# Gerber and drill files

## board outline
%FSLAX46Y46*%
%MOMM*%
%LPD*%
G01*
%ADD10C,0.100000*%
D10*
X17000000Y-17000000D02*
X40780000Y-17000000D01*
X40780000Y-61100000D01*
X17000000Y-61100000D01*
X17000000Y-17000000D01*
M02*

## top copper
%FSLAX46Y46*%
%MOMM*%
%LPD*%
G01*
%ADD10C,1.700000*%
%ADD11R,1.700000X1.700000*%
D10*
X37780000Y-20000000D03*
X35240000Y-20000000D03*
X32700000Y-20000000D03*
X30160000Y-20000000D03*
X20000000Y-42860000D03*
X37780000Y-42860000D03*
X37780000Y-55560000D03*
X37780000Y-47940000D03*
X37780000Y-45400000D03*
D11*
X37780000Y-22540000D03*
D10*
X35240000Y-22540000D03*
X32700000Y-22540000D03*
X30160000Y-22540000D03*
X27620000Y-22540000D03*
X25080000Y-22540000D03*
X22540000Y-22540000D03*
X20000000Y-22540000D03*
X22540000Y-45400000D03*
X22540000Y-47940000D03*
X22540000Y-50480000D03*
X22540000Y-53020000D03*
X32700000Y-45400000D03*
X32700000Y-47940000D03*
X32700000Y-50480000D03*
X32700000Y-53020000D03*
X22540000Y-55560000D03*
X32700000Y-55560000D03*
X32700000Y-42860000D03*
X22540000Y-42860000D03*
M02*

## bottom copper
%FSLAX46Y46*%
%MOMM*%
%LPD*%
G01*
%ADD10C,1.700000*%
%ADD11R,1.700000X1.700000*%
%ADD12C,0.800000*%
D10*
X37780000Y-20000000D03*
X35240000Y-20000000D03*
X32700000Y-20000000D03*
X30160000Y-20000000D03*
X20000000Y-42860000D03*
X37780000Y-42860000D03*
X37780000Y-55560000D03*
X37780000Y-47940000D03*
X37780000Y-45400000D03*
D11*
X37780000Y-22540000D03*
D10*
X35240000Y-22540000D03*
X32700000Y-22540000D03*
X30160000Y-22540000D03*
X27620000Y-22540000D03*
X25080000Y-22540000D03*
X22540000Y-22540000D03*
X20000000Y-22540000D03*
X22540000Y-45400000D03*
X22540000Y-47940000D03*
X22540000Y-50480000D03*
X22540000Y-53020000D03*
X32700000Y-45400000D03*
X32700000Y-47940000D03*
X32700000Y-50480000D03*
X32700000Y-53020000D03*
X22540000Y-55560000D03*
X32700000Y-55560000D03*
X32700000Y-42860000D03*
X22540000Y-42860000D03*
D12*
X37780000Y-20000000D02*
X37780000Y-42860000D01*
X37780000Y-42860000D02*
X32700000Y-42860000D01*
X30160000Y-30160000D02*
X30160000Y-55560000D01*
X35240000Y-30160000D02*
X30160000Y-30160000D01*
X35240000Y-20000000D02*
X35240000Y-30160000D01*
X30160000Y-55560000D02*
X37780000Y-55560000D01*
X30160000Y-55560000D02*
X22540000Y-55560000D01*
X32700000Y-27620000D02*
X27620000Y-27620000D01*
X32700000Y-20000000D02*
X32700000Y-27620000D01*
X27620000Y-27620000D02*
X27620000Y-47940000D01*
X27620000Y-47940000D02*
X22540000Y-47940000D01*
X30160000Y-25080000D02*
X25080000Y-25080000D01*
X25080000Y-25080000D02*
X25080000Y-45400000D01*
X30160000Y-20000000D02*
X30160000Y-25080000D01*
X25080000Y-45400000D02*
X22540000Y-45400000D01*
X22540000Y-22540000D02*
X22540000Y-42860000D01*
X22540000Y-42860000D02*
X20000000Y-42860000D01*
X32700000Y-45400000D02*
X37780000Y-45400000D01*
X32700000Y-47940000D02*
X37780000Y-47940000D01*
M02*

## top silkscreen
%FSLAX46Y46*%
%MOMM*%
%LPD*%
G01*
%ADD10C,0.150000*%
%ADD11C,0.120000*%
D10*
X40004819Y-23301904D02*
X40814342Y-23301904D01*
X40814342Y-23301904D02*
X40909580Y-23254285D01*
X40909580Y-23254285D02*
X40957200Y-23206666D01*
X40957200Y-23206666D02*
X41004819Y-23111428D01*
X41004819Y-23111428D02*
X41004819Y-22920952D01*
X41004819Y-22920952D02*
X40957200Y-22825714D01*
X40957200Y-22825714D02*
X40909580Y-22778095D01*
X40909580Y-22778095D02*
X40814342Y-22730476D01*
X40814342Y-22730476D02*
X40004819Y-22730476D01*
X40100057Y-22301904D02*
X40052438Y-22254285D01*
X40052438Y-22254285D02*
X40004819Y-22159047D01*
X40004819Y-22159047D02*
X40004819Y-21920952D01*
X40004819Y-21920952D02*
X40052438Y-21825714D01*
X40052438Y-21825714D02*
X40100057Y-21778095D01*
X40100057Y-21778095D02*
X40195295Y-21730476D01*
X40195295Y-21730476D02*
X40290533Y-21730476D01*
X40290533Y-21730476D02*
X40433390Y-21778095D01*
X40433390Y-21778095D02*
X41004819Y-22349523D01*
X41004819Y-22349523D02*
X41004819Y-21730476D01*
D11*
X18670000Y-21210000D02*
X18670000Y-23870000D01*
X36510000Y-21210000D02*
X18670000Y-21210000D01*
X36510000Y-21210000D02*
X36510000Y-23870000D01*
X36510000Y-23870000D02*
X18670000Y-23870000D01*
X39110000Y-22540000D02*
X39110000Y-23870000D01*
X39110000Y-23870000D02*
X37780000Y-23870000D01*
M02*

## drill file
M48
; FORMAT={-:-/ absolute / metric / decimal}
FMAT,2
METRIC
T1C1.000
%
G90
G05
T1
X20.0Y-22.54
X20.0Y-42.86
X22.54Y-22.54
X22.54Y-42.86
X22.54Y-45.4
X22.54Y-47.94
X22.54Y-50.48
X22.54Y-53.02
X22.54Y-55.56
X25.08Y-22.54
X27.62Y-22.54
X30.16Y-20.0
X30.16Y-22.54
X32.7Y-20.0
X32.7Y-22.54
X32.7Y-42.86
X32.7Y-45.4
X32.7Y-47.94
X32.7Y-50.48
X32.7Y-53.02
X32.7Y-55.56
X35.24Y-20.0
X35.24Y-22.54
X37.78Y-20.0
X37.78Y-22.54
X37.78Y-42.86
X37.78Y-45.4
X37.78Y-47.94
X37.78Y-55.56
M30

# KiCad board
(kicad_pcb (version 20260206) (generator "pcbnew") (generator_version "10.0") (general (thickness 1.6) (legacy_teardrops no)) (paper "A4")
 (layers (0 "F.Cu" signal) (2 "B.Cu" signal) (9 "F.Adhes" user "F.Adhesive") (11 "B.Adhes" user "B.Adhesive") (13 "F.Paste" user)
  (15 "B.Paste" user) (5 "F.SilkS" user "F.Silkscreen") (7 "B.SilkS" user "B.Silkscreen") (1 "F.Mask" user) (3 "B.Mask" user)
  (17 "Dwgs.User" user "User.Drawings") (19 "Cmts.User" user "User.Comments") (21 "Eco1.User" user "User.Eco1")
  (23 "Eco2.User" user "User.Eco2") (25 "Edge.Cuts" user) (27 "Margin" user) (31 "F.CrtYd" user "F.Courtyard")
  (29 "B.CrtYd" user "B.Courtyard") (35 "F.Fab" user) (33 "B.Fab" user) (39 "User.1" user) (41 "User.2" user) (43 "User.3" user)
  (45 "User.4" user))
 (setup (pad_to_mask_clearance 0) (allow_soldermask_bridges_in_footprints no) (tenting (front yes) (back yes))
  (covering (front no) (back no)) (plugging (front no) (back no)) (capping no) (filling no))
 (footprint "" (layer "F.Cu") (at 30.16 20)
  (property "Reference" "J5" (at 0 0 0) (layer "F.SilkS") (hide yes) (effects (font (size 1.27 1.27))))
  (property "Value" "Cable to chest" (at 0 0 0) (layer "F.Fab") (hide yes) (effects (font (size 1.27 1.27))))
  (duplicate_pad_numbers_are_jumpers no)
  (pad "c5V" thru_hole circle (at 7.62 0) (size 1.7 1.7) (drill 1) (layers "*.Cu" "*.Mask") (remove_unused_layers no) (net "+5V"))
  (pad "cGND" thru_hole circle (at 5.08 0) (size 1.7 1.7) (drill 1) (layers "*.Cu" "*.Mask") (remove_unused_layers no) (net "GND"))
  (pad "cSCL" thru_hole circle (at 2.54 0) (size 1.7 1.7) (drill 1) (layers "*.Cu" "*.Mask") (remove_unused_layers no) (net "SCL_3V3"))
  (pad "cSDA" thru_hole circle (at 0 0) (size 1.7 1.7) (drill 1) (layers "*.Cu" "*.Mask") (remove_unused_layers no) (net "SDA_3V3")))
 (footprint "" (layer "F.Cu") (at 20 42.86)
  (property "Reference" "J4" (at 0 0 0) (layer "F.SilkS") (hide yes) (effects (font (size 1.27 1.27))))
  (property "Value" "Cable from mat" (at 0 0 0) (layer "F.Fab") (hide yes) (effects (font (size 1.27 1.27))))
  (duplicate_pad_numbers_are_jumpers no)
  (pad "m3V3" thru_hole circle (at 0 0) (size 1.7 1.7) (drill 1) (layers "*.Cu" "*.Mask") (remove_unused_layers no) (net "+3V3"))
  (pad "m5V" thru_hole circle (at 17.78 0) (size 1.7 1.7) (drill 1) (layers "*.Cu" "*.Mask") (remove_unused_layers no) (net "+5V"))
  (pad "mGND" thru_hole circle (at 17.78 12.7) (size 1.7 1.7) (drill 1) (layers "*.Cu" "*.Mask") (remove_unused_layers no) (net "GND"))
  (pad "mSCL" thru_hole circle (at 17.78 5.08) (size 1.7 1.7) (drill 1) (layers "*.Cu" "*.Mask") (remove_unused_layers no) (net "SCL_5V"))
  (pad "mSDA" thru_hole circle (at 17.78 2.54) (size 1.7 1.7) (drill 1) (layers "*.Cu" "*.Mask") (remove_unused_layers no) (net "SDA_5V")))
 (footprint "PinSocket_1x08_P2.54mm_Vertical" (layer "F.Cu") (at 37.78 22.54 -90)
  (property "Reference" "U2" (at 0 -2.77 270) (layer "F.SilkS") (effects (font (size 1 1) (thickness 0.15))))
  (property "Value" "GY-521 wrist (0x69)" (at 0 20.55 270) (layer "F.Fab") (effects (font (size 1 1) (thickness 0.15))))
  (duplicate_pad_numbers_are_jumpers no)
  (fp_line (start -1.33 19.11) (end 1.33 19.11) (stroke (width 0.12) (type solid)) (layer "F.SilkS"))
  (fp_line (start -1.33 1.27) (end -1.33 19.11) (stroke (width 0.12) (type solid)) (layer "F.SilkS"))
  (fp_line (start -1.33 1.27) (end 1.33 1.27) (stroke (width 0.12) (type solid)) (layer "F.SilkS"))
  (fp_line (start 1.33 1.27) (end 1.33 19.11) (stroke (width 0.12) (type solid)) (layer "F.SilkS"))
  (fp_line (start 0 -1.33) (end 1.33 -1.33) (stroke (width 0.12) (type solid)) (layer "F.SilkS"))
  (fp_line (start 1.33 -1.33) (end 1.33 0) (stroke (width 0.12) (type solid)) (layer "F.SilkS"))
  (pad "1" thru_hole rect (at 0 0 270) (size 1.7 1.7) (drill 1) (layers "*.Cu" "*.Mask") (remove_unused_layers no) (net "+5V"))
  (pad "2" thru_hole circle (at 0 2.54 270) (size 1.7 1.7) (drill 1) (layers "*.Cu" "*.Mask") (remove_unused_layers no) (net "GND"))
  (pad "3" thru_hole circle (at 0 5.08 270) (size 1.7 1.7) (drill 1) (layers "*.Cu" "*.Mask") (remove_unused_layers no) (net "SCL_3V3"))
  (pad "4" thru_hole circle (at 0 7.62 270) (size 1.7 1.7) (drill 1) (layers "*.Cu" "*.Mask") (remove_unused_layers no) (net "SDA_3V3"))
  (pad "5" thru_hole circle (at 0 10.16 270) (size 1.7 1.7) (drill 1) (layers "*.Cu" "*.Mask") (remove_unused_layers no))
  (pad "6" thru_hole circle (at 0 12.7 270) (size 1.7 1.7) (drill 1) (layers "*.Cu" "*.Mask") (remove_unused_layers no))
  (pad "7" thru_hole circle (at 0 15.24 270) (size 1.7 1.7) (drill 1) (layers "*.Cu" "*.Mask") (remove_unused_layers no) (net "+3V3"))
  (pad "8" thru_hole circle (at 0 17.78 270) (size 1.7 1.7) (drill 1) (layers "*.Cu" "*.Mask") (remove_unused_layers no)))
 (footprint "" (layer "F.Cu") (at 22.54 42.86)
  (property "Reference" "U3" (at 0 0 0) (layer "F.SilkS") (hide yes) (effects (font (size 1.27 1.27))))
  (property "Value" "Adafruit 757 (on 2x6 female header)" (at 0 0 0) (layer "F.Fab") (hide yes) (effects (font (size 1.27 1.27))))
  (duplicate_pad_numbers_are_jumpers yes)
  (pad "A1" thru_hole circle (at 0 2.54) (size 1.7 1.7) (drill 1) (layers "*.Cu" "*.Mask") (remove_unused_layers no) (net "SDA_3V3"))
  (pad "A2" thru_hole circle (at 0 5.08) (size 1.7 1.7) (drill 1) (layers "*.Cu" "*.Mask") (remove_unused_layers no) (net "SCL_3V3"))
  (pad "A3" thru_hole circle (at 0 7.62) (size 1.7 1.7) (drill 1) (layers "*.Cu" "*.Mask") (remove_unused_layers no))
  (pad "A4" thru_hole circle (at 0 10.16) (size 1.7 1.7) (drill 1) (layers "*.Cu" "*.Mask") (remove_unused_layers no))
  (pad "B1" thru_hole circle (at 10.16 2.54) (size 1.7 1.7) (drill 1) (layers "*.Cu" "*.Mask") (remove_unused_layers no) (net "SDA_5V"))
  (pad "B2" thru_hole circle (at 10.16 5.08) (size 1.7 1.7) (drill 1) (layers "*.Cu" "*.Mask") (remove_unused_layers no) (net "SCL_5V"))
  (pad "B3" thru_hole circle (at 10.16 7.62) (size 1.7 1.7) (drill 1) (layers "*.Cu" "*.Mask") (remove_unused_layers no))
  (pad "B4" thru_hole circle (at 10.16 10.16) (size 1.7 1.7) (drill 1) (layers "*.Cu" "*.Mask") (remove_unused_layers no))
  (pad "GND" thru_hole circle (at 0 12.7) (size 1.7 1.7) (drill 1) (layers "*.Cu" "*.Mask") (remove_unused_layers no) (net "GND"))
  (pad "GND" thru_hole circle (at 10.16 12.7) (size 1.7 1.7) (drill 1) (layers "*.Cu" "*.Mask") (remove_unused_layers no) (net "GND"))
  (pad "HV" thru_hole circle (at 10.16 0) (size 1.7 1.7) (drill 1) (layers "*.Cu" "*.Mask") (remove_unused_layers no) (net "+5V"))
  (pad "LV" thru_hole circle (at 0 0) (size 1.7 1.7) (drill 1) (layers "*.Cu" "*.Mask") (remove_unused_layers no) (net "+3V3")))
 (gr_rect (start 17 17) (end 40.78 61.1) (stroke (width 0.1) (type default)) (fill no) (layer "Edge.Cuts"))
 (segment (start 37.78 20) (end 37.78 42.86) (width 0.8) (layer "B.Cu") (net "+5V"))
 (segment (start 37.78 42.86) (end 32.7 42.86) (width 0.8) (layer "B.Cu") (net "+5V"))
 (segment (start 30.16 30.16) (end 30.16 55.56) (width 0.8) (layer "B.Cu") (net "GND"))
 (segment (start 35.24 30.16) (end 30.16 30.16) (width 0.8) (layer "B.Cu") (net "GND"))
 (segment (start 35.24 20) (end 35.24 30.16) (width 0.8) (layer "B.Cu") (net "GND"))
 (segment (start 30.16 55.56) (end 37.78 55.56) (width 0.8) (layer "B.Cu") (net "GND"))
 (segment (start 30.16 55.56) (end 22.54 55.56) (width 0.8) (layer "B.Cu") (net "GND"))
 (segment (start 32.7 27.62) (end 27.62 27.62) (width 0.8) (layer "B.Cu") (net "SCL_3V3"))
 (segment (start 32.7 20) (end 32.7 27.62) (width 0.8) (layer "B.Cu") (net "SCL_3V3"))
 (segment (start 27.62 27.62) (end 27.62 47.94) (width 0.8) (layer "B.Cu") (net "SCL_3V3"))
 (segment (start 27.62 47.94) (end 22.54 47.94) (width 0.8) (layer "B.Cu") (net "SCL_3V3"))
 (segment (start 30.16 25.08) (end 25.08 25.08) (width 0.8) (layer "B.Cu") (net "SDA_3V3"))
 (segment (start 25.08 25.08) (end 25.08 45.4) (width 0.8) (layer "B.Cu") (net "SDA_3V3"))
 (segment (start 30.16 20) (end 30.16 25.08) (width 0.8) (layer "B.Cu") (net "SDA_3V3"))
 (segment (start 25.08 45.4) (end 22.54 45.4) (width 0.8) (layer "B.Cu") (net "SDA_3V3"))
 (segment (start 22.54 22.54) (end 22.54 42.86) (width 0.8) (layer "B.Cu") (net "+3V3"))
 (segment (start 22.54 42.86) (end 20 42.86) (width 0.8) (layer "B.Cu") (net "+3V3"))
 (segment (start 32.7 45.4) (end 37.78 45.4) (width 0.8) (layer "B.Cu") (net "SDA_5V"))
 (segment (start 32.7 47.94) (end 37.78 47.94) (width 0.8) (layer "B.Cu") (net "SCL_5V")))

